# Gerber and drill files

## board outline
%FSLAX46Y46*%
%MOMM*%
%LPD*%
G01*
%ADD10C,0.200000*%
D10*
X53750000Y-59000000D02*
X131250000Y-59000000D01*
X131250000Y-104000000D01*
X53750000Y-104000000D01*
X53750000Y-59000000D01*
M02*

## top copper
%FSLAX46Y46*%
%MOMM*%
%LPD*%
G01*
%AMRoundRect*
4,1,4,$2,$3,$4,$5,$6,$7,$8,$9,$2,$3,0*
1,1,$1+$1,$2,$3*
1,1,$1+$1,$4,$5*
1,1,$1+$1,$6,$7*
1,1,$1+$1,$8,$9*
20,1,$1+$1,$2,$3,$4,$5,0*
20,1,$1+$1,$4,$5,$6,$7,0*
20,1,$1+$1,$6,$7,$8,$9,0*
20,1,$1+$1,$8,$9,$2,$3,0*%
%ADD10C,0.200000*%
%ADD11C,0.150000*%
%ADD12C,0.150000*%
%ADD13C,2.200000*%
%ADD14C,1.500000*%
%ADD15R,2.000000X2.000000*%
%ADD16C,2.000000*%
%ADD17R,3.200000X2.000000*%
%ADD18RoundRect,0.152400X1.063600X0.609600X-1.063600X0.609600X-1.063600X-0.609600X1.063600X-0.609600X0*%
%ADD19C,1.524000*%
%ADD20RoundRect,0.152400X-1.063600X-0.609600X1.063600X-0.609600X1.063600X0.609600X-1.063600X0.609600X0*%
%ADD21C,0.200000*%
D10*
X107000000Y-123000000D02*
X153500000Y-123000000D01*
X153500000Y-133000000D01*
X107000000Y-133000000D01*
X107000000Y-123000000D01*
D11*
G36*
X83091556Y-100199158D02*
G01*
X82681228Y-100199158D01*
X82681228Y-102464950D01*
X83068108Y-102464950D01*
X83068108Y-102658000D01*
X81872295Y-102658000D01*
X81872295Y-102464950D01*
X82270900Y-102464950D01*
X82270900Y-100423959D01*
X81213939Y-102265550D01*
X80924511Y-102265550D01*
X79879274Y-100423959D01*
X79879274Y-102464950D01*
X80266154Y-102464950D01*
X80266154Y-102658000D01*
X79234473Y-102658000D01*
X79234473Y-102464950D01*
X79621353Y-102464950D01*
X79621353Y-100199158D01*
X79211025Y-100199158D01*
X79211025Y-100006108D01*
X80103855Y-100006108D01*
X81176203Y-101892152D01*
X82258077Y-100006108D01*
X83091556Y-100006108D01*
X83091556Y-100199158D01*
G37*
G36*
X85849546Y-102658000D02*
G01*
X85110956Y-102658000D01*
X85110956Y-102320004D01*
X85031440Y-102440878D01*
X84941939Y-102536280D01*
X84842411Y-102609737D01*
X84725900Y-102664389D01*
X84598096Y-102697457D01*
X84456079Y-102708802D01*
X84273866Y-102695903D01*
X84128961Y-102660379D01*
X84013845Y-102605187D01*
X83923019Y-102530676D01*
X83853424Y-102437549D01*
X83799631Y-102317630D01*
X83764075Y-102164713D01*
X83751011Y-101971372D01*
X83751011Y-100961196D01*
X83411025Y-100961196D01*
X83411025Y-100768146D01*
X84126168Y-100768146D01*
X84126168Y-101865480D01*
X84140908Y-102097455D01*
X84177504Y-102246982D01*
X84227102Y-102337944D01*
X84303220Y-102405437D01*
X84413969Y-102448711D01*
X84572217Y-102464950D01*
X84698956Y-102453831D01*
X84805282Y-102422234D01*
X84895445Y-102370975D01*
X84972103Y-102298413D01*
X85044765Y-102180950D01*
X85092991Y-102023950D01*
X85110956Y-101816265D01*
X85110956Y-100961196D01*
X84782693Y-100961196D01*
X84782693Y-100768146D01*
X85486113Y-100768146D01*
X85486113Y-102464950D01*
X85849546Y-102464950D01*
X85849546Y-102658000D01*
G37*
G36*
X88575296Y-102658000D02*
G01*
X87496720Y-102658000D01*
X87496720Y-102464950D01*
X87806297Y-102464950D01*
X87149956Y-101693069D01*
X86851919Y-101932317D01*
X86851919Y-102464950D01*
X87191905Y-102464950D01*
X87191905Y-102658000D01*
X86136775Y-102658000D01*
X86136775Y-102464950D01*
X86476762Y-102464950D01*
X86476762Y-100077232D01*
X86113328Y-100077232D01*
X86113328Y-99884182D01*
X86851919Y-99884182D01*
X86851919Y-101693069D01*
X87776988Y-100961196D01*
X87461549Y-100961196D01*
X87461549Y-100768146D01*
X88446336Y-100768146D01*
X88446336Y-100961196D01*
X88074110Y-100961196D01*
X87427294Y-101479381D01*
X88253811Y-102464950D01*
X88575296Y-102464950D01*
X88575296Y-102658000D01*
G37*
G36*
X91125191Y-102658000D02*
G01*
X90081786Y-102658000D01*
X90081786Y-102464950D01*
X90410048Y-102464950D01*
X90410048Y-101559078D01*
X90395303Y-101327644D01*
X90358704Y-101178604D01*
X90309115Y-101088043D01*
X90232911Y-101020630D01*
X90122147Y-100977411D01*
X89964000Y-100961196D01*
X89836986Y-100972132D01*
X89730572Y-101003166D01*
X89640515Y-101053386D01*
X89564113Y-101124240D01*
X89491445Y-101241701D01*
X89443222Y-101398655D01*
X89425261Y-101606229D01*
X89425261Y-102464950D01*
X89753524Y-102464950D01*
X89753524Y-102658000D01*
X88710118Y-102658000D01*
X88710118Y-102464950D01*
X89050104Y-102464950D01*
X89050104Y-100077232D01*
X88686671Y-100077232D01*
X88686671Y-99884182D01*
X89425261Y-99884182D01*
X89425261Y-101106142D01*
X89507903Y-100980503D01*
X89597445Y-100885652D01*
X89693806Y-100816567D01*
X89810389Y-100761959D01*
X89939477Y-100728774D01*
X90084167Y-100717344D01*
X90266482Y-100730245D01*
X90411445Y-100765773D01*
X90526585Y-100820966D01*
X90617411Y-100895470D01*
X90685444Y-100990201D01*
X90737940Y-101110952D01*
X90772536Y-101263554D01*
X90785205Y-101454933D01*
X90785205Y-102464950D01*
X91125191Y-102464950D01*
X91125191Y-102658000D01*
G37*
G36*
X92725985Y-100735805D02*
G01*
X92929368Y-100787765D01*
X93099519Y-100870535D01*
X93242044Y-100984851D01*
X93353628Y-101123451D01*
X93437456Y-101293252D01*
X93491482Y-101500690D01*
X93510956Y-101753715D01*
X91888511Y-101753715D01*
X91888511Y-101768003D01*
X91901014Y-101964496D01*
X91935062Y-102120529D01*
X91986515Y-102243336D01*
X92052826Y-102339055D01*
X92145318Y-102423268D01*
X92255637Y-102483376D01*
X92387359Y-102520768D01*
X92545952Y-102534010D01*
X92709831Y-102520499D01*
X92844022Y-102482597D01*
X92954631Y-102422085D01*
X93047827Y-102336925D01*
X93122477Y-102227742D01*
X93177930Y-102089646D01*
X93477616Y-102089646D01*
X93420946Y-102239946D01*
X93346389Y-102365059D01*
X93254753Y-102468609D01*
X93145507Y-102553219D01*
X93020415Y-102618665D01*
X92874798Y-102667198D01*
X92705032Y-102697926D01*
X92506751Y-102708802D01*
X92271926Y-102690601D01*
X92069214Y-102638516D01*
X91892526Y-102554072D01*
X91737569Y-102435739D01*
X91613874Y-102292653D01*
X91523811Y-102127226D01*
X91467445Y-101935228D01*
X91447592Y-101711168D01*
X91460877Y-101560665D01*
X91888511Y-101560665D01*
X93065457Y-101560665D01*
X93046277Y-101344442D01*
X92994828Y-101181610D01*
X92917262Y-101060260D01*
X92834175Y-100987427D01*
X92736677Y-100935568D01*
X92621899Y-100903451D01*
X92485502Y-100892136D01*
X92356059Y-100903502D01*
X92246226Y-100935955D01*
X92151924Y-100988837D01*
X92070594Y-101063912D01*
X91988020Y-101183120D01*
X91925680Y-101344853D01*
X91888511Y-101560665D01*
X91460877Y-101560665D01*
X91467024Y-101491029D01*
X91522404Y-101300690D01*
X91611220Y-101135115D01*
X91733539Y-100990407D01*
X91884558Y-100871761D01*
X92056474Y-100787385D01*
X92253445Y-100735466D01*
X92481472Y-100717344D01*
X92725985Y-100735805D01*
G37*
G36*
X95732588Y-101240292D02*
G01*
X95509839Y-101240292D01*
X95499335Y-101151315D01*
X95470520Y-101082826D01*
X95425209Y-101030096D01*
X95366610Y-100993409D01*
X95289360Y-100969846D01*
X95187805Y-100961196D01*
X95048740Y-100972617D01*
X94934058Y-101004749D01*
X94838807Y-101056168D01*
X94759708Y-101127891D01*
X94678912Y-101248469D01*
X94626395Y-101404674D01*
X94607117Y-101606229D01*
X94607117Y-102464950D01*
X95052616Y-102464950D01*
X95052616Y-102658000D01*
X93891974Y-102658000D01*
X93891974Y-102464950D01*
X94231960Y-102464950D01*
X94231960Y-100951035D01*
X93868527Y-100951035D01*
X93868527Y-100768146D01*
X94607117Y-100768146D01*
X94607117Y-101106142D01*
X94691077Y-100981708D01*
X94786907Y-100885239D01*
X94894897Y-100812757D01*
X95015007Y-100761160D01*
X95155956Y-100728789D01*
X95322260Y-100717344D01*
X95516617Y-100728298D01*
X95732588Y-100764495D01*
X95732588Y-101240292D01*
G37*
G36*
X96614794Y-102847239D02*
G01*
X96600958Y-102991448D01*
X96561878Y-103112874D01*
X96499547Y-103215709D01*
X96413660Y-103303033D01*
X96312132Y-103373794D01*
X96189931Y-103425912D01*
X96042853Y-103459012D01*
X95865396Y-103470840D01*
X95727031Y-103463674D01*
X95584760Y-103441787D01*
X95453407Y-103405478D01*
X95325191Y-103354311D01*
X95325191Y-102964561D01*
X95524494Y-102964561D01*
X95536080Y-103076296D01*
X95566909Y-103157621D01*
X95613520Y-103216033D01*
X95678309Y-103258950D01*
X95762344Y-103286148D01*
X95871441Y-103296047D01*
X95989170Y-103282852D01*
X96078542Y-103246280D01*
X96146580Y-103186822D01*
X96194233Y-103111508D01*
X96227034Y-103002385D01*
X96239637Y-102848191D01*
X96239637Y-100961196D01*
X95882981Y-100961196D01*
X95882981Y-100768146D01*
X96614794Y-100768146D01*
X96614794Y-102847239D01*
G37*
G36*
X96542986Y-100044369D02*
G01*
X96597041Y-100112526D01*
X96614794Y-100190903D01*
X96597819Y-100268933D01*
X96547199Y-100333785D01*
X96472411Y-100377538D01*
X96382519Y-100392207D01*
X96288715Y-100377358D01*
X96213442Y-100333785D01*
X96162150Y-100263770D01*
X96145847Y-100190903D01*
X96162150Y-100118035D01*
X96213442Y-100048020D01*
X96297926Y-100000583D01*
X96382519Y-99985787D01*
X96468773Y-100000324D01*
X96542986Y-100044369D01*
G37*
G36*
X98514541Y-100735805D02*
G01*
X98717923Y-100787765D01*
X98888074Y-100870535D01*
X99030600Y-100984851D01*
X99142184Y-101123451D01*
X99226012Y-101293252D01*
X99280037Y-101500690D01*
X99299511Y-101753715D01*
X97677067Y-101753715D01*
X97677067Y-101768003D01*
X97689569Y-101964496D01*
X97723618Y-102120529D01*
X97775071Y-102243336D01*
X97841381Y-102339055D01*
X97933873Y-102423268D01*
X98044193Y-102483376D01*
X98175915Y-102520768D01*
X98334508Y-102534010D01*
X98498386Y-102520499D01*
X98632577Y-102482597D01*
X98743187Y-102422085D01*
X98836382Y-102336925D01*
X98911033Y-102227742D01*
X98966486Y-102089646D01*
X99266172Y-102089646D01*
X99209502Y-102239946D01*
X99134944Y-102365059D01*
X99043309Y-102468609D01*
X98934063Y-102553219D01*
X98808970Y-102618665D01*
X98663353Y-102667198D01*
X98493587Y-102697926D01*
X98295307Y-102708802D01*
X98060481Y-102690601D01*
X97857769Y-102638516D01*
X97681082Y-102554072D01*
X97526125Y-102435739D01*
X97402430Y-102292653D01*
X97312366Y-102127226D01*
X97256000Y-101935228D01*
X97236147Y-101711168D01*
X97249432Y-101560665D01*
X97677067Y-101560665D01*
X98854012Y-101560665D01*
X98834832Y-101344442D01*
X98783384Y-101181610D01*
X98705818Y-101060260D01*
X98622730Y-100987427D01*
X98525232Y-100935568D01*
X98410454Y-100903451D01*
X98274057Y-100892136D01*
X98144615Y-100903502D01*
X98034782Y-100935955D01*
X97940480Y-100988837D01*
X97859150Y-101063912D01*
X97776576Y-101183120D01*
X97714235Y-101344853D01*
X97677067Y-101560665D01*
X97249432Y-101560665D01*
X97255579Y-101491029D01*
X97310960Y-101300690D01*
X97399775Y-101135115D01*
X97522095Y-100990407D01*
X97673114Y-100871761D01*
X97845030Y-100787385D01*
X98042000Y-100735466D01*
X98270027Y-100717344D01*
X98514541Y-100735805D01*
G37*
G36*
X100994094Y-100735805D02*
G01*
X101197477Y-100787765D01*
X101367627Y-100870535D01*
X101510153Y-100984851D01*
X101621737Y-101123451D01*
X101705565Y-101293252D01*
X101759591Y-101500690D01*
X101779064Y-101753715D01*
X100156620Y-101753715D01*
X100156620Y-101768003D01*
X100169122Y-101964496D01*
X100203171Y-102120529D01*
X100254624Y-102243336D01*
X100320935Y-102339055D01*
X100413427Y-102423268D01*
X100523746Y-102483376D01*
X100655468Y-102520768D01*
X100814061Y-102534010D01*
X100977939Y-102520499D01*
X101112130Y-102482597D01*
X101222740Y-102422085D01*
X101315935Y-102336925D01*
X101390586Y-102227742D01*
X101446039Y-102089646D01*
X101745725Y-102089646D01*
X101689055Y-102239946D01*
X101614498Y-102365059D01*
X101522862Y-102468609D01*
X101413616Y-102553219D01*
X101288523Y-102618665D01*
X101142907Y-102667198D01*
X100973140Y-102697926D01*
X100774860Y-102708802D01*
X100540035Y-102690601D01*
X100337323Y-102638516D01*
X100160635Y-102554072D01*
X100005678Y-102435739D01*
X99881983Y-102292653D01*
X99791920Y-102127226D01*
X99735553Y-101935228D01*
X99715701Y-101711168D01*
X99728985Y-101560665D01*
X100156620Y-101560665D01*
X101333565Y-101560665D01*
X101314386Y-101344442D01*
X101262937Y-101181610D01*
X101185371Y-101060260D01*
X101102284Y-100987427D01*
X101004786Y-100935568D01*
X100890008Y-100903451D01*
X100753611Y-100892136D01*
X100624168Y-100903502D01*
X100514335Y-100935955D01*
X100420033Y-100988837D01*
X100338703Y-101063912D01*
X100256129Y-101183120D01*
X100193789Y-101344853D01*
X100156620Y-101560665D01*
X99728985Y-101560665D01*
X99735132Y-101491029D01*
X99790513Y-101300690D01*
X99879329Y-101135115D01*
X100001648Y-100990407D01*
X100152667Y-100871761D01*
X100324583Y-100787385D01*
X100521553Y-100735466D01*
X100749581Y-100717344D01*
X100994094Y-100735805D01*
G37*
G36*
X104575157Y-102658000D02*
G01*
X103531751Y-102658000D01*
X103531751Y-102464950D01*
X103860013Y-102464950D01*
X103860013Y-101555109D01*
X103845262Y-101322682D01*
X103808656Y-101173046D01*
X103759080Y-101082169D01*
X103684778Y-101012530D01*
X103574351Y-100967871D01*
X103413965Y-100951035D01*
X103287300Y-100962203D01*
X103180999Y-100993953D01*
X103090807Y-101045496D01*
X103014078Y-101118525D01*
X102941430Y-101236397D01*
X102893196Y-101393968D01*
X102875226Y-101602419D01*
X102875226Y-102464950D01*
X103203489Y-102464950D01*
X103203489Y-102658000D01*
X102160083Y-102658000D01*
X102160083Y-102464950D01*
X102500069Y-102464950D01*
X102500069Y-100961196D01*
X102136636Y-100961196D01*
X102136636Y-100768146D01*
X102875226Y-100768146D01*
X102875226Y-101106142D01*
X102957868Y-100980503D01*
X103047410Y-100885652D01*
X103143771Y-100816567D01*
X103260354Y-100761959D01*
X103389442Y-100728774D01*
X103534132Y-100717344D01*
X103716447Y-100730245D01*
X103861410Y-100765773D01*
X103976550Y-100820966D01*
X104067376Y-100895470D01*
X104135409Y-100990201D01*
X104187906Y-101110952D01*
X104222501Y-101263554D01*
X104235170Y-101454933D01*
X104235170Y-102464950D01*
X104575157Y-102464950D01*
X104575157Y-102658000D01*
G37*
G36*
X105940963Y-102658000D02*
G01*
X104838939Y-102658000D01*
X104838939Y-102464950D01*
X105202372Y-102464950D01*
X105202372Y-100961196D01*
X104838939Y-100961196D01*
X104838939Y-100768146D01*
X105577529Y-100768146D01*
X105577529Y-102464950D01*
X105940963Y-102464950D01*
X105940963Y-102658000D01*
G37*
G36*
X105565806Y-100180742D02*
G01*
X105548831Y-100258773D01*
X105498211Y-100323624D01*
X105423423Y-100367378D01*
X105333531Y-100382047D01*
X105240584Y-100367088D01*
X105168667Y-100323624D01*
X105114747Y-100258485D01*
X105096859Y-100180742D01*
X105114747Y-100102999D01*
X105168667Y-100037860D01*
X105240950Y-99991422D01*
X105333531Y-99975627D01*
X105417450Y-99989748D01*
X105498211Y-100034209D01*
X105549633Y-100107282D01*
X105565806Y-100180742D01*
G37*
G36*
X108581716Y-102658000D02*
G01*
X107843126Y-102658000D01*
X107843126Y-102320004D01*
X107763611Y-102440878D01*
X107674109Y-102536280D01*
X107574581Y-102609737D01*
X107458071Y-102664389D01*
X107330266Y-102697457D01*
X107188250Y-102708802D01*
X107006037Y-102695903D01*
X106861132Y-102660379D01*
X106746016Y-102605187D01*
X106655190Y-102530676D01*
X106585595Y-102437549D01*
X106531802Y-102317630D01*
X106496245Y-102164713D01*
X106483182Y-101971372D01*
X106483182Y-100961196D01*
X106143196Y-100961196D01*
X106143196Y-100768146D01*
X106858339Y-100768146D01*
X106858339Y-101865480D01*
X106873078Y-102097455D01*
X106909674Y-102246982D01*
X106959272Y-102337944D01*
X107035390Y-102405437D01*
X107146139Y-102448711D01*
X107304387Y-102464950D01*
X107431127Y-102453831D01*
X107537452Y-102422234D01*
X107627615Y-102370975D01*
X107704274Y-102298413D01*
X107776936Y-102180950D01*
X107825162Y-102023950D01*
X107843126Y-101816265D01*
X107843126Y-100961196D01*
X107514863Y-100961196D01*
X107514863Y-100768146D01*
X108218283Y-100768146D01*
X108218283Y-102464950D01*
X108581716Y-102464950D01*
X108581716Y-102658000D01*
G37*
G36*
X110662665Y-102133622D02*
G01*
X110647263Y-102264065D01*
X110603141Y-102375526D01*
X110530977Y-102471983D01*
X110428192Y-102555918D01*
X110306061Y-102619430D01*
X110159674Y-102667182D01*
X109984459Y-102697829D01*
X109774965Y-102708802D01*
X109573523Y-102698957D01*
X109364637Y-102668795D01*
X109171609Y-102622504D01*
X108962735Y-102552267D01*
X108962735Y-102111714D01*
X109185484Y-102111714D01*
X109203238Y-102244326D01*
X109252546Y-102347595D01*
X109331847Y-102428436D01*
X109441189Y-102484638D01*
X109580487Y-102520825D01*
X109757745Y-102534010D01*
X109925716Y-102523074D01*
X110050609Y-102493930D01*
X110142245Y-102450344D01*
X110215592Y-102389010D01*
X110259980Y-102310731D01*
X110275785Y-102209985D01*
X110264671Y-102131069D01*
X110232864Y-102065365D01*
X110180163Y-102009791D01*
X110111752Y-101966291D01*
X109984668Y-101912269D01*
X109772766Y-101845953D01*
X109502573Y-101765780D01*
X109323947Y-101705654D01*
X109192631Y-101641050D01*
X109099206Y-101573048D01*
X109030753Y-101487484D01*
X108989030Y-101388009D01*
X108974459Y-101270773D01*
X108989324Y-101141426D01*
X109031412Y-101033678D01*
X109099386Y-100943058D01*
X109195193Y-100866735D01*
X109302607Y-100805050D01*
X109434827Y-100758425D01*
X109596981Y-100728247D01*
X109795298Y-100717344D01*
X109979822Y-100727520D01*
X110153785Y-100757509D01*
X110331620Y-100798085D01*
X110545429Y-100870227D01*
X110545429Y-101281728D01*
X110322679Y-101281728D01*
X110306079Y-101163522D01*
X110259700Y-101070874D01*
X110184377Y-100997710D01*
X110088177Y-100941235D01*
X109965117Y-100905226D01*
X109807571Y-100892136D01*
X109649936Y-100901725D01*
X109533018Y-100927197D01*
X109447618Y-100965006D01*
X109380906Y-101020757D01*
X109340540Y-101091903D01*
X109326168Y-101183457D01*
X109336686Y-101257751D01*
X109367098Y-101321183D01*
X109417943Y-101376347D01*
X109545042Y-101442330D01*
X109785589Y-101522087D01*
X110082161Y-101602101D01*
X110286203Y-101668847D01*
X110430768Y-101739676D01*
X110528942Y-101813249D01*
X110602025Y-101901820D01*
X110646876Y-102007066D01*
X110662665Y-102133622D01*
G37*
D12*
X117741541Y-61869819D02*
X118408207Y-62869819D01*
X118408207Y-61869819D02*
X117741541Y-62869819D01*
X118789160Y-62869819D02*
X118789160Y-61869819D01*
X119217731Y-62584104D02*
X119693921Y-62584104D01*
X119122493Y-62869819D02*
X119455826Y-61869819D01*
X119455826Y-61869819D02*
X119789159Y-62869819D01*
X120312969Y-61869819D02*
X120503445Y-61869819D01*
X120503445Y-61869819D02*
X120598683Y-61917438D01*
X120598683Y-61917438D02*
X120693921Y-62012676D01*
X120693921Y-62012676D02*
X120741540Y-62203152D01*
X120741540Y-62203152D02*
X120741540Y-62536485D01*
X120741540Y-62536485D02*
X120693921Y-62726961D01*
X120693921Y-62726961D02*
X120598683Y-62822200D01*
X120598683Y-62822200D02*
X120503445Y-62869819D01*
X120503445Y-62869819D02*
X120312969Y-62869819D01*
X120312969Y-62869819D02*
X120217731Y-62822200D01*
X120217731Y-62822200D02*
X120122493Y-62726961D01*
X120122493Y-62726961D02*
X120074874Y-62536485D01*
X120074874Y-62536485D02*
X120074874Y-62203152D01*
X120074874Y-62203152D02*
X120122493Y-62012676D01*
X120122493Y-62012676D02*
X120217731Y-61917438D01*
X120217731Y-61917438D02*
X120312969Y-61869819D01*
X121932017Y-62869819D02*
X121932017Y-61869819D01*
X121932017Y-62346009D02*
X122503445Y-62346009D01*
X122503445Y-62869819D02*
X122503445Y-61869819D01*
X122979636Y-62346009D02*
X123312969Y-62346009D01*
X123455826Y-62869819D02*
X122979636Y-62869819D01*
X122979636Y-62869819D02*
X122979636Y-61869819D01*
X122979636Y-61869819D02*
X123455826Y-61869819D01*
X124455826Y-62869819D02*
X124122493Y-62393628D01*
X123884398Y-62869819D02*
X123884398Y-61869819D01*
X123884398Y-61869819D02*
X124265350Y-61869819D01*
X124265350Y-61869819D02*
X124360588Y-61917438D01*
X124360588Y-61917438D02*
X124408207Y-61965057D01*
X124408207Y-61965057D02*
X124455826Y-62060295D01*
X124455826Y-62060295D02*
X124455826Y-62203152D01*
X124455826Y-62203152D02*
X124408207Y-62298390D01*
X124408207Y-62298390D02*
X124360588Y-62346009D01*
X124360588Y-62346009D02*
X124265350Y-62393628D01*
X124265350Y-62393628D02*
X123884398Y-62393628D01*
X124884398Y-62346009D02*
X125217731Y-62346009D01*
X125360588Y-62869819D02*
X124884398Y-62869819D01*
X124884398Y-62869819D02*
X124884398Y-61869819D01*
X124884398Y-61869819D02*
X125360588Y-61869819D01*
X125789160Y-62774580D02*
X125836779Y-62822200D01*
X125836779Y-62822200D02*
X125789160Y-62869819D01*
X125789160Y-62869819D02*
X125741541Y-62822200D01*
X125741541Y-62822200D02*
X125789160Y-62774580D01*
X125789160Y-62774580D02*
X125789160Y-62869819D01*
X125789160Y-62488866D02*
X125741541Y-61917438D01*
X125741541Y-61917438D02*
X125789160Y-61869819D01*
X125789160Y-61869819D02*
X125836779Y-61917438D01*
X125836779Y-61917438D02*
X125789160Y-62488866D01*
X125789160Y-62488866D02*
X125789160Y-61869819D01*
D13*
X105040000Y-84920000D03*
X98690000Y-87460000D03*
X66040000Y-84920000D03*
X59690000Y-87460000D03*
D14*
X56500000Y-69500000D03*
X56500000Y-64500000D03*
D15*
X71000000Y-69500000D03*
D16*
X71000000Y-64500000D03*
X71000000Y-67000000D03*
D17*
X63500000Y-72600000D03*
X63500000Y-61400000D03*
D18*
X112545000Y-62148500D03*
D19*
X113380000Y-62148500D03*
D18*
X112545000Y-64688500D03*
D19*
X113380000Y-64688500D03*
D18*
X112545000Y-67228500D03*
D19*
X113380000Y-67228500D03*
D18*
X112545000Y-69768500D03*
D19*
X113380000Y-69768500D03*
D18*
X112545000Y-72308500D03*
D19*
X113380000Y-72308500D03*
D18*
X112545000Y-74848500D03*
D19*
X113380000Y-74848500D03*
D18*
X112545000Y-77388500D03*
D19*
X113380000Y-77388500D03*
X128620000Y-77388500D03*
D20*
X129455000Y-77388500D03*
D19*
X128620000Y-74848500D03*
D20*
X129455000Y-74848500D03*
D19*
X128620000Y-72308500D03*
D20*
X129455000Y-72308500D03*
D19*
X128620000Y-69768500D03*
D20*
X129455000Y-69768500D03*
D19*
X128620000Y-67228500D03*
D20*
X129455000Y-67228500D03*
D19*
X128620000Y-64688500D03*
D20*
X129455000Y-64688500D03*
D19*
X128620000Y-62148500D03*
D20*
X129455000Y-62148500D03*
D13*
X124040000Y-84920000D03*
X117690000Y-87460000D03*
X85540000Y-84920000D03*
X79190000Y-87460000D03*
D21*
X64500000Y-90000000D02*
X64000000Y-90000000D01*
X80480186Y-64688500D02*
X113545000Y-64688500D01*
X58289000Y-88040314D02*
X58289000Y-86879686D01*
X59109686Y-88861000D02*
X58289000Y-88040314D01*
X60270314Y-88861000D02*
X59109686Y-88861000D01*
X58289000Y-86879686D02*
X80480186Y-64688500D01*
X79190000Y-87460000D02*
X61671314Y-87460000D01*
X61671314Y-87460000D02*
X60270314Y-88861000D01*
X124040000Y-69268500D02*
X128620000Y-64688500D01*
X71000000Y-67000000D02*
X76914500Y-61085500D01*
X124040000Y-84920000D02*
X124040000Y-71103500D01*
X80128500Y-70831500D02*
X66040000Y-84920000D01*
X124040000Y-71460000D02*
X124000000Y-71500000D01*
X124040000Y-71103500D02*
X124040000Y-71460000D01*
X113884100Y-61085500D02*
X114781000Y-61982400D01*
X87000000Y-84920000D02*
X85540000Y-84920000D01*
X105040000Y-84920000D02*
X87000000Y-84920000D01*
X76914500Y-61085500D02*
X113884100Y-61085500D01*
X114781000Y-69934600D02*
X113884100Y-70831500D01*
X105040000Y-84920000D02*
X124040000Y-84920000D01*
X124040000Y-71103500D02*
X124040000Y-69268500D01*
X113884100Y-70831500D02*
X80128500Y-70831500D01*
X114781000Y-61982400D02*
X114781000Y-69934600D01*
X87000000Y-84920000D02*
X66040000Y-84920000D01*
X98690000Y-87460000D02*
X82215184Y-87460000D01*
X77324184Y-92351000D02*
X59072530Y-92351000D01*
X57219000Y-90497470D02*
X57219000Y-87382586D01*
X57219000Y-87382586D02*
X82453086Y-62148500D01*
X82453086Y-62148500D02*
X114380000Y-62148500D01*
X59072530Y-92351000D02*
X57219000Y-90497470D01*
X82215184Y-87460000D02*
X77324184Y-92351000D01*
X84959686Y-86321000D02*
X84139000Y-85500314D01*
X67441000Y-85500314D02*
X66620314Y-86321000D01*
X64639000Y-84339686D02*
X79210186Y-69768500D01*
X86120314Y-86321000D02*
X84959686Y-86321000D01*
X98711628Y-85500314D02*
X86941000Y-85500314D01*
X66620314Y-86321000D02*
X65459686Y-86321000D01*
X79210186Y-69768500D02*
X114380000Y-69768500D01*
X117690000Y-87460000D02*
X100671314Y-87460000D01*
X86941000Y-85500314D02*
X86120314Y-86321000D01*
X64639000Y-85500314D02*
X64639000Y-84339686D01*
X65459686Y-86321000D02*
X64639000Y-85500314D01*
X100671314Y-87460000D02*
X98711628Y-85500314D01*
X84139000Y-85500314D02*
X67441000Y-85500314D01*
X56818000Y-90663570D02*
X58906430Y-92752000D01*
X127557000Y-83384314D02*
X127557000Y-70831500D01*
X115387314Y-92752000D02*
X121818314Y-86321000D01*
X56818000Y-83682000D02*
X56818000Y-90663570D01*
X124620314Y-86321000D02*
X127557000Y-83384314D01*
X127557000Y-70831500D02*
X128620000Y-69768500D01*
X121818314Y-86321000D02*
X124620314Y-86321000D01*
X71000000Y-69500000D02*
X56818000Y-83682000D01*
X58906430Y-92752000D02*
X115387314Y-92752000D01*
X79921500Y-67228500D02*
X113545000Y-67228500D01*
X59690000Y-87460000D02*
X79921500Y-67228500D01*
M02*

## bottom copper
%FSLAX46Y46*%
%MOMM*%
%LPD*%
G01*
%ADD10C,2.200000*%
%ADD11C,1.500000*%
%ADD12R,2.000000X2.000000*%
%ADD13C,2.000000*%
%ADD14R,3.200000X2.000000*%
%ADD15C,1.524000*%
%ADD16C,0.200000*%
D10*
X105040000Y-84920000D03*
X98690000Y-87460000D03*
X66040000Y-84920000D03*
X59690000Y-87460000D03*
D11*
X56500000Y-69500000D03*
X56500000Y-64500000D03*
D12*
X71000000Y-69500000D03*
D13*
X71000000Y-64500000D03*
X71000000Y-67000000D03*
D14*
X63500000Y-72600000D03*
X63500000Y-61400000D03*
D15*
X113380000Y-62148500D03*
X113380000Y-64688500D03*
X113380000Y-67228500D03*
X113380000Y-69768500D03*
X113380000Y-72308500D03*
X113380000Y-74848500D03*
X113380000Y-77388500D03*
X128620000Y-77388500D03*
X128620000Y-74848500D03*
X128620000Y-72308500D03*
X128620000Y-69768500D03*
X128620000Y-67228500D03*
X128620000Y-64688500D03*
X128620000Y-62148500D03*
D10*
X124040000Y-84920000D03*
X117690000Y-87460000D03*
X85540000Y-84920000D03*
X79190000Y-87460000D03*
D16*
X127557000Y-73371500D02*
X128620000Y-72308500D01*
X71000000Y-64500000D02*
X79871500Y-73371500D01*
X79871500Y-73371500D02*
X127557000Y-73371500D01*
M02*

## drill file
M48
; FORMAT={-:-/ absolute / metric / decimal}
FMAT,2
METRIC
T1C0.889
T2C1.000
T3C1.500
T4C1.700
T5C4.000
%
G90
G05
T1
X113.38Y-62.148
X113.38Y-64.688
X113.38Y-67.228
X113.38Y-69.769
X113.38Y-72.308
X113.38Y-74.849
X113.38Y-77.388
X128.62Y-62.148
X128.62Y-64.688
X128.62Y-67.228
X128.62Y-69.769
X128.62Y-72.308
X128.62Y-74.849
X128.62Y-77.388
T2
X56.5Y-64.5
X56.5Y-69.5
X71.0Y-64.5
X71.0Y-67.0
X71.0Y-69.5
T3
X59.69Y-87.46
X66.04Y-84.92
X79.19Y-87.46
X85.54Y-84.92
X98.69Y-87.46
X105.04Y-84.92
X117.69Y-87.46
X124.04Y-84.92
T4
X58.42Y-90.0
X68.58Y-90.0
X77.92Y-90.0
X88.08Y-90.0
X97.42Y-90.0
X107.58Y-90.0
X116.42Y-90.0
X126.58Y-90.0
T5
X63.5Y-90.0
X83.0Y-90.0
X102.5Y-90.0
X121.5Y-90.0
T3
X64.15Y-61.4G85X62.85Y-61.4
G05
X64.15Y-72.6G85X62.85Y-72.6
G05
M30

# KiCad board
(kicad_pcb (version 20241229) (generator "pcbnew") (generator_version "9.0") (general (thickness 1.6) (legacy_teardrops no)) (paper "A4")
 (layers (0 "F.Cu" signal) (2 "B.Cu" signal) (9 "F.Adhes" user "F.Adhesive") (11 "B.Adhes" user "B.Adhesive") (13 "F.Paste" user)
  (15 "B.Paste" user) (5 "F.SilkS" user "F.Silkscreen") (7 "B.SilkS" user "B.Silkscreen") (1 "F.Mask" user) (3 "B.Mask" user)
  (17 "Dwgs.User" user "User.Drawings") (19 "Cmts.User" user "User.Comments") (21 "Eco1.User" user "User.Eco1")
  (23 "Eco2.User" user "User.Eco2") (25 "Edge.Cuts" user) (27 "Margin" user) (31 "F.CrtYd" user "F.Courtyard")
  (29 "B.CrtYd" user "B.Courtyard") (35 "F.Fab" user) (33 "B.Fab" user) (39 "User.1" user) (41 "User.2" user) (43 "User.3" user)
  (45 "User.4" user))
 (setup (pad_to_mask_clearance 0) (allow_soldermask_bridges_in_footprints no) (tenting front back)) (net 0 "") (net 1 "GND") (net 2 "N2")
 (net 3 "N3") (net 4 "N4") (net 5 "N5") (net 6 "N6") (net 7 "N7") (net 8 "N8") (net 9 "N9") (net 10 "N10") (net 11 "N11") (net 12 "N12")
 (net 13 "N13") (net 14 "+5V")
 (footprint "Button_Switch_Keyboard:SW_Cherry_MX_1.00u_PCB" (layer "F.Cu") (at 105.04 84.92)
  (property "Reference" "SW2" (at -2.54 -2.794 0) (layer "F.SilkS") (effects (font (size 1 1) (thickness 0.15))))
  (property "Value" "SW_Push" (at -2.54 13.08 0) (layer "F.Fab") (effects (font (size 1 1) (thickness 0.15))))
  (pad "" np_thru_hole circle (at -7.62 5.08) (size 1.7 1.7) (drill 1.7) (layers "*.Cu" "*.Mask"))
  (pad "" np_thru_hole circle (at -2.54 5.08) (size 4 4) (drill 4) (layers "*.Cu" "*.Mask"))
  (pad "" np_thru_hole circle (at 2.54 5.08) (size 1.7 1.7) (drill 1.7) (layers "*.Cu" "*.Mask"))
  (pad "1" thru_hole circle (at 0 0) (size 2.2 2.2) (drill 1.5) (layers "*.Cu" "*.Mask") (remove_unused_layers no) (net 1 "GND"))
  (pad "2" thru_hole circle (at -6.35 2.54) (size 2.2 2.2) (drill 1.5) (layers "*.Cu" "*.Mask") (remove_unused_layers no) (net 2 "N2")))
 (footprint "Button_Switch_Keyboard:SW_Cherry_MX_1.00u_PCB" (layer "F.Cu") (at 66.04 84.92)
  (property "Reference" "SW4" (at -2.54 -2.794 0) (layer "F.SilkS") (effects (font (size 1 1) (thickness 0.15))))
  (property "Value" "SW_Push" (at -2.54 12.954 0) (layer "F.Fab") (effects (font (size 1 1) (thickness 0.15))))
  (pad "" np_thru_hole circle (at -7.62 5.08) (size 1.7 1.7) (drill 1.7) (layers "*.Cu" "*.Mask"))
  (pad "" np_thru_hole circle (at -2.54 5.08) (size 4 4) (drill 4) (layers "*.Cu" "*.Mask"))
  (pad "" np_thru_hole circle (at 2.54 5.08) (size 1.7 1.7) (drill 1.7) (layers "*.Cu" "*.Mask"))
  (pad "1" thru_hole circle (at 0 0) (size 2.2 2.2) (drill 1.5) (layers "*.Cu" "*.Mask") (remove_unused_layers no) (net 1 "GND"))
  (pad "2" thru_hole circle (at -6.35 2.54) (size 2.2 2.2) (drill 1.5) (layers "*.Cu" "*.Mask") (remove_unused_layers no) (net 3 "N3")))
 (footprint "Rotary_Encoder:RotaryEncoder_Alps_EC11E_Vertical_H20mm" (layer "F.Cu") (at 71 69.5 180)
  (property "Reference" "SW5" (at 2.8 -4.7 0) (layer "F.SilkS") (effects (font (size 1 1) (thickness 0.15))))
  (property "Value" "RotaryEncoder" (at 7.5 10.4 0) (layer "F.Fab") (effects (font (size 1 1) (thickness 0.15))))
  (pad "" thru_hole circle (at 14.5 0 180) (size 1.5 1.5) (drill 1) (layers "*.Cu" "*.Mask") (remove_unused_layers no))
  (pad "" thru_hole circle (at 14.5 5 180) (size 1.5 1.5) (drill 1) (layers "*.Cu" "*.Mask") (remove_unused_layers no))
  (pad "A" thru_hole rect (at 0 0 180) (size 2 2) (drill 1) (layers "*.Cu" "*.Mask") (remove_unused_layers no) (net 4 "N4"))
  (pad "B" thru_hole circle (at 0 5 180) (size 2 2) (drill 1) (layers "*.Cu" "*.Mask") (remove_unused_layers no) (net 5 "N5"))
  (pad "C" thru_hole circle (at 0 2.5 180) (size 2 2) (drill 1) (layers "*.Cu" "*.Mask") (remove_unused_layers no) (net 1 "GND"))
  (pad "MP" thru_hole rect (at 7.5 -3.1 180) (size 3.2 2) (drill oval 2.8 1.5) (layers "*.Cu" "*.Mask") (remove_unused_layers no))
  (pad "MP" thru_hole rect (at 7.5 8.1 180) (size 3.2 2) (drill oval 2.8 1.5) (layers "*.Cu" "*.Mask") (remove_unused_layers no)))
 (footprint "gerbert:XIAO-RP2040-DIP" (layer "F.Cu") (at 121 69.7685)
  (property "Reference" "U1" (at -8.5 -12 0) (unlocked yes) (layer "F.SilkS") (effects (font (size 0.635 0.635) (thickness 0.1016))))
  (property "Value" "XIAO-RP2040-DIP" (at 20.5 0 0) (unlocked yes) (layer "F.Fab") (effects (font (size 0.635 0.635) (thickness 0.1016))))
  (pad "1" smd roundrect (at -8.455 -7.62 180) (size 2.432 1.524) (layers "F.Cu" "F.Mask") (roundrect_rratio 0.1) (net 2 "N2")
   (thermal_bridge_angle 45))
  (pad "1" thru_hole circle (at -7.62 -7.62 180) (size 1.524 1.524) (drill 0.889) (layers "*.Cu" "*.Mask") (remove_unused_layers no)
   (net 2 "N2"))
  (pad "2" smd roundrect (at -8.455 -5.08 180) (size 2.432 1.524) (layers "F.Cu" "F.Mask") (roundrect_rratio 0.1) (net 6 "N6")
   (thermal_bridge_angle 45))
  (pad "2" thru_hole circle (at -7.62 -5.08 180) (size 1.524 1.524) (drill 0.889) (layers "*.Cu" "*.Mask") (remove_unused_layers no)
   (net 6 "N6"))
  (pad "3" smd roundrect (at -8.455 -2.54 180) (size 2.432 1.524) (layers "F.Cu" "F.Mask") (roundrect_rratio 0.1) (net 3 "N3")
   (thermal_bridge_angle 45))
  (pad "3" thru_hole circle (at -7.62 -2.54 180) (size 1.524 1.524) (drill 0.889) (layers "*.Cu" "*.Mask") (remove_unused_layers no)
   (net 3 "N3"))
  (pad "4" smd roundrect (at -8.455 0 180) (size 2.432 1.524) (layers "F.Cu" "F.Mask") (roundrect_rratio 0.1) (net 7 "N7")
   (thermal_bridge_angle 45))
  (pad "4" thru_hole circle (at -7.62 0 180) (size 1.524 1.524) (drill 0.889) (layers "*.Cu" "*.Mask") (remove_unused_layers no)
   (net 7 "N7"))
  (pad "5" smd roundrect (at -8.455 2.54 180) (size 2.432 1.524) (layers "F.Cu" "F.Mask") (roundrect_rratio 0.1) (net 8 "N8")
   (thermal_bridge_angle 45))
  (pad "5" thru_hole circle (at -7.62 2.54 180) (size 1.524 1.524) (drill 0.889) (layers "*.Cu" "*.Mask") (remove_unused_layers no)
   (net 8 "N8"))
  (pad "6" smd roundrect (at -8.455 5.08 180) (size 2.432 1.524) (layers "F.Cu" "F.Mask") (roundrect_rratio 0.1) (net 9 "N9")
   (thermal_bridge_angle 45))
  (pad "6" thru_hole circle (at -7.62 5.08 180) (size 1.524 1.524) (drill 0.889) (layers "*.Cu" "*.Mask") (remove_unused_layers no)
   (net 9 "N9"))
  (pad "7" smd roundrect (at -8.455 7.62 180) (size 2.432 1.524) (layers "F.Cu" "F.Mask") (roundrect_rratio 0.1) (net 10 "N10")
   (thermal_bridge_angle 45))
  (pad "7" thru_hole circle (at -7.62 7.62 180) (size 1.524 1.524) (drill 0.889) (layers "*.Cu" "*.Mask") (remove_unused_layers no)
   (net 10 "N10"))
  (pad "8" thru_hole circle (at 7.62 7.62) (size 1.524 1.524) (drill 0.889) (layers "*.Cu" "*.Mask") (remove_unused_layers no)
   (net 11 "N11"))
  (pad "8" smd roundrect (at 8.455 7.62) (size 2.432 1.524) (layers "F.Cu" "F.Mask") (roundrect_rratio 0.1) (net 11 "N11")
   (thermal_bridge_angle 45))
  (pad "9" thru_hole circle (at 7.62 5.08) (size 1.524 1.524) (drill 0.889) (layers "*.Cu" "*.Mask") (remove_unused_layers no)
   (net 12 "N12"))
  (pad "9" smd roundrect (at 8.455 5.08) (size 2.432 1.524) (layers "F.Cu" "F.Mask") (roundrect_rratio 0.1) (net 12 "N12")
   (thermal_bridge_angle 45))
  (pad "10" thru_hole circle (at 7.62 2.54) (size 1.524 1.524) (drill 0.889) (layers "*.Cu" "*.Mask") (remove_unused_layers no) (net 5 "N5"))
  (pad "10" smd roundrect (at 8.455 2.54) (size 2.432 1.524) (layers "F.Cu" "F.Mask") (roundrect_rratio 0.1) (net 5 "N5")
   (thermal_bridge_angle 45))
  (pad "11" thru_hole circle (at 7.62 0) (size 1.524 1.524) (drill 0.889) (layers "*.Cu" "*.Mask") (remove_unused_layers no) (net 4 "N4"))
  (pad "11" smd roundrect (at 8.455 0) (size 2.432 1.524) (layers "F.Cu" "F.Mask") (roundrect_rratio 0.1) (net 4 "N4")
   (thermal_bridge_angle 45))
  (pad "12" thru_hole circle (at 7.62 -2.54) (size 1.524 1.524) (drill 0.889) (layers "*.Cu" "*.Mask") (remove_unused_layers no)
   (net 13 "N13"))
  (pad "12" smd roundrect (at 8.455 -2.54) (size 2.432 1.524) (layers "F.Cu" "F.Mask") (roundrect_rratio 0.1) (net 13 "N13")
   (thermal_bridge_angle 45))
  (pad "13" thru_hole circle (at 7.62 -5.08) (size 1.524 1.524) (drill 0.889) (layers "*.Cu" "*.Mask") (remove_unused_layers no)
   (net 1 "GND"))
  (pad "13" smd roundrect (at 8.455 -5.08) (size 2.432 1.524) (layers "F.Cu" "F.Mask") (roundrect_rratio 0.1) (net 1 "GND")
   (thermal_bridge_angle 45))
  (pad "14" thru_hole circle (at 7.62 -7.62) (size 1.524 1.524) (drill 0.889) (layers "*.Cu" "*.Mask") (remove_unused_layers no)
   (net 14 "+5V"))
  (pad "14" smd roundrect (at 8.455 -7.62) (size 2.432 1.524) (layers "F.Cu" "F.Mask") (roundrect_rratio 0.1) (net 14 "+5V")
   (thermal_bridge_angle 45)))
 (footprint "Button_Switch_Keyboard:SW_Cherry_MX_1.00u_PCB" (layer "F.Cu") (at 124.04 84.92)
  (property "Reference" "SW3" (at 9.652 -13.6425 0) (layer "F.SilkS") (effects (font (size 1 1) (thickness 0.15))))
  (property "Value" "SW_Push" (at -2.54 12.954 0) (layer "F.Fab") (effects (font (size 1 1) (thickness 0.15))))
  (pad "" np_thru_hole circle (at -7.62 5.08) (size 1.7 1.7) (drill 1.7) (layers "*.Cu" "*.Mask"))
  (pad "" np_thru_hole circle (at -2.54 5.08) (size 4 4) (drill 4) (layers "*.Cu" "*.Mask"))
  (pad "" np_thru_hole circle (at 2.54 5.08) (size 1.7 1.7) (drill 1.7) (layers "*.Cu" "*.Mask"))
  (pad "1" thru_hole circle (at 0 0) (size 2.2 2.2) (drill 1.5) (layers "*.Cu" "*.Mask") (remove_unused_layers no) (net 1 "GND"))
  (pad "2" thru_hole circle (at -6.35 2.54) (size 2.2 2.2) (drill 1.5) (layers "*.Cu" "*.Mask") (remove_unused_layers no) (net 7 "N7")))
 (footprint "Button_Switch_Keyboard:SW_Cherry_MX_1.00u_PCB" (layer "F.Cu") (at 85.54 84.92)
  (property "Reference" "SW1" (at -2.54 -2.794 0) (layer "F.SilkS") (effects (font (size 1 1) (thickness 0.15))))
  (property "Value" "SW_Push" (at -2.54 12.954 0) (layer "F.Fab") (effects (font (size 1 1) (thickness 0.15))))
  (pad "" np_thru_hole circle (at -7.62 5.08) (size 1.7 1.7) (drill 1.7) (layers "*.Cu" "*.Mask"))
  (pad "" np_thru_hole circle (at -2.54 5.08) (size 4 4) (drill 4) (layers "*.Cu" "*.Mask"))
  (pad "" np_thru_hole circle (at 2.54 5.08) (size 1.7 1.7) (drill 1.7) (layers "*.Cu" "*.Mask"))
  (pad "1" thru_hole circle (at 0 0) (size 2.2 2.2) (drill 1.5) (layers "*.Cu" "*.Mask") (remove_unused_layers no) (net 1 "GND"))
  (pad "2" thru_hole circle (at -6.35 2.54) (size 2.2 2.2) (drill 1.5) (layers "*.Cu" "*.Mask") (remove_unused_layers no) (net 6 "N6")))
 (gr_rect (start 107 123) (end 153.5 133) (stroke (width 0.2) (type default)) (fill no) (layer "F.Cu"))
 (gr_rect (start 53.75 59) (end 131.25 104) (stroke (width 0.2) (type solid)) (fill no) (layer "Edge.Cuts"))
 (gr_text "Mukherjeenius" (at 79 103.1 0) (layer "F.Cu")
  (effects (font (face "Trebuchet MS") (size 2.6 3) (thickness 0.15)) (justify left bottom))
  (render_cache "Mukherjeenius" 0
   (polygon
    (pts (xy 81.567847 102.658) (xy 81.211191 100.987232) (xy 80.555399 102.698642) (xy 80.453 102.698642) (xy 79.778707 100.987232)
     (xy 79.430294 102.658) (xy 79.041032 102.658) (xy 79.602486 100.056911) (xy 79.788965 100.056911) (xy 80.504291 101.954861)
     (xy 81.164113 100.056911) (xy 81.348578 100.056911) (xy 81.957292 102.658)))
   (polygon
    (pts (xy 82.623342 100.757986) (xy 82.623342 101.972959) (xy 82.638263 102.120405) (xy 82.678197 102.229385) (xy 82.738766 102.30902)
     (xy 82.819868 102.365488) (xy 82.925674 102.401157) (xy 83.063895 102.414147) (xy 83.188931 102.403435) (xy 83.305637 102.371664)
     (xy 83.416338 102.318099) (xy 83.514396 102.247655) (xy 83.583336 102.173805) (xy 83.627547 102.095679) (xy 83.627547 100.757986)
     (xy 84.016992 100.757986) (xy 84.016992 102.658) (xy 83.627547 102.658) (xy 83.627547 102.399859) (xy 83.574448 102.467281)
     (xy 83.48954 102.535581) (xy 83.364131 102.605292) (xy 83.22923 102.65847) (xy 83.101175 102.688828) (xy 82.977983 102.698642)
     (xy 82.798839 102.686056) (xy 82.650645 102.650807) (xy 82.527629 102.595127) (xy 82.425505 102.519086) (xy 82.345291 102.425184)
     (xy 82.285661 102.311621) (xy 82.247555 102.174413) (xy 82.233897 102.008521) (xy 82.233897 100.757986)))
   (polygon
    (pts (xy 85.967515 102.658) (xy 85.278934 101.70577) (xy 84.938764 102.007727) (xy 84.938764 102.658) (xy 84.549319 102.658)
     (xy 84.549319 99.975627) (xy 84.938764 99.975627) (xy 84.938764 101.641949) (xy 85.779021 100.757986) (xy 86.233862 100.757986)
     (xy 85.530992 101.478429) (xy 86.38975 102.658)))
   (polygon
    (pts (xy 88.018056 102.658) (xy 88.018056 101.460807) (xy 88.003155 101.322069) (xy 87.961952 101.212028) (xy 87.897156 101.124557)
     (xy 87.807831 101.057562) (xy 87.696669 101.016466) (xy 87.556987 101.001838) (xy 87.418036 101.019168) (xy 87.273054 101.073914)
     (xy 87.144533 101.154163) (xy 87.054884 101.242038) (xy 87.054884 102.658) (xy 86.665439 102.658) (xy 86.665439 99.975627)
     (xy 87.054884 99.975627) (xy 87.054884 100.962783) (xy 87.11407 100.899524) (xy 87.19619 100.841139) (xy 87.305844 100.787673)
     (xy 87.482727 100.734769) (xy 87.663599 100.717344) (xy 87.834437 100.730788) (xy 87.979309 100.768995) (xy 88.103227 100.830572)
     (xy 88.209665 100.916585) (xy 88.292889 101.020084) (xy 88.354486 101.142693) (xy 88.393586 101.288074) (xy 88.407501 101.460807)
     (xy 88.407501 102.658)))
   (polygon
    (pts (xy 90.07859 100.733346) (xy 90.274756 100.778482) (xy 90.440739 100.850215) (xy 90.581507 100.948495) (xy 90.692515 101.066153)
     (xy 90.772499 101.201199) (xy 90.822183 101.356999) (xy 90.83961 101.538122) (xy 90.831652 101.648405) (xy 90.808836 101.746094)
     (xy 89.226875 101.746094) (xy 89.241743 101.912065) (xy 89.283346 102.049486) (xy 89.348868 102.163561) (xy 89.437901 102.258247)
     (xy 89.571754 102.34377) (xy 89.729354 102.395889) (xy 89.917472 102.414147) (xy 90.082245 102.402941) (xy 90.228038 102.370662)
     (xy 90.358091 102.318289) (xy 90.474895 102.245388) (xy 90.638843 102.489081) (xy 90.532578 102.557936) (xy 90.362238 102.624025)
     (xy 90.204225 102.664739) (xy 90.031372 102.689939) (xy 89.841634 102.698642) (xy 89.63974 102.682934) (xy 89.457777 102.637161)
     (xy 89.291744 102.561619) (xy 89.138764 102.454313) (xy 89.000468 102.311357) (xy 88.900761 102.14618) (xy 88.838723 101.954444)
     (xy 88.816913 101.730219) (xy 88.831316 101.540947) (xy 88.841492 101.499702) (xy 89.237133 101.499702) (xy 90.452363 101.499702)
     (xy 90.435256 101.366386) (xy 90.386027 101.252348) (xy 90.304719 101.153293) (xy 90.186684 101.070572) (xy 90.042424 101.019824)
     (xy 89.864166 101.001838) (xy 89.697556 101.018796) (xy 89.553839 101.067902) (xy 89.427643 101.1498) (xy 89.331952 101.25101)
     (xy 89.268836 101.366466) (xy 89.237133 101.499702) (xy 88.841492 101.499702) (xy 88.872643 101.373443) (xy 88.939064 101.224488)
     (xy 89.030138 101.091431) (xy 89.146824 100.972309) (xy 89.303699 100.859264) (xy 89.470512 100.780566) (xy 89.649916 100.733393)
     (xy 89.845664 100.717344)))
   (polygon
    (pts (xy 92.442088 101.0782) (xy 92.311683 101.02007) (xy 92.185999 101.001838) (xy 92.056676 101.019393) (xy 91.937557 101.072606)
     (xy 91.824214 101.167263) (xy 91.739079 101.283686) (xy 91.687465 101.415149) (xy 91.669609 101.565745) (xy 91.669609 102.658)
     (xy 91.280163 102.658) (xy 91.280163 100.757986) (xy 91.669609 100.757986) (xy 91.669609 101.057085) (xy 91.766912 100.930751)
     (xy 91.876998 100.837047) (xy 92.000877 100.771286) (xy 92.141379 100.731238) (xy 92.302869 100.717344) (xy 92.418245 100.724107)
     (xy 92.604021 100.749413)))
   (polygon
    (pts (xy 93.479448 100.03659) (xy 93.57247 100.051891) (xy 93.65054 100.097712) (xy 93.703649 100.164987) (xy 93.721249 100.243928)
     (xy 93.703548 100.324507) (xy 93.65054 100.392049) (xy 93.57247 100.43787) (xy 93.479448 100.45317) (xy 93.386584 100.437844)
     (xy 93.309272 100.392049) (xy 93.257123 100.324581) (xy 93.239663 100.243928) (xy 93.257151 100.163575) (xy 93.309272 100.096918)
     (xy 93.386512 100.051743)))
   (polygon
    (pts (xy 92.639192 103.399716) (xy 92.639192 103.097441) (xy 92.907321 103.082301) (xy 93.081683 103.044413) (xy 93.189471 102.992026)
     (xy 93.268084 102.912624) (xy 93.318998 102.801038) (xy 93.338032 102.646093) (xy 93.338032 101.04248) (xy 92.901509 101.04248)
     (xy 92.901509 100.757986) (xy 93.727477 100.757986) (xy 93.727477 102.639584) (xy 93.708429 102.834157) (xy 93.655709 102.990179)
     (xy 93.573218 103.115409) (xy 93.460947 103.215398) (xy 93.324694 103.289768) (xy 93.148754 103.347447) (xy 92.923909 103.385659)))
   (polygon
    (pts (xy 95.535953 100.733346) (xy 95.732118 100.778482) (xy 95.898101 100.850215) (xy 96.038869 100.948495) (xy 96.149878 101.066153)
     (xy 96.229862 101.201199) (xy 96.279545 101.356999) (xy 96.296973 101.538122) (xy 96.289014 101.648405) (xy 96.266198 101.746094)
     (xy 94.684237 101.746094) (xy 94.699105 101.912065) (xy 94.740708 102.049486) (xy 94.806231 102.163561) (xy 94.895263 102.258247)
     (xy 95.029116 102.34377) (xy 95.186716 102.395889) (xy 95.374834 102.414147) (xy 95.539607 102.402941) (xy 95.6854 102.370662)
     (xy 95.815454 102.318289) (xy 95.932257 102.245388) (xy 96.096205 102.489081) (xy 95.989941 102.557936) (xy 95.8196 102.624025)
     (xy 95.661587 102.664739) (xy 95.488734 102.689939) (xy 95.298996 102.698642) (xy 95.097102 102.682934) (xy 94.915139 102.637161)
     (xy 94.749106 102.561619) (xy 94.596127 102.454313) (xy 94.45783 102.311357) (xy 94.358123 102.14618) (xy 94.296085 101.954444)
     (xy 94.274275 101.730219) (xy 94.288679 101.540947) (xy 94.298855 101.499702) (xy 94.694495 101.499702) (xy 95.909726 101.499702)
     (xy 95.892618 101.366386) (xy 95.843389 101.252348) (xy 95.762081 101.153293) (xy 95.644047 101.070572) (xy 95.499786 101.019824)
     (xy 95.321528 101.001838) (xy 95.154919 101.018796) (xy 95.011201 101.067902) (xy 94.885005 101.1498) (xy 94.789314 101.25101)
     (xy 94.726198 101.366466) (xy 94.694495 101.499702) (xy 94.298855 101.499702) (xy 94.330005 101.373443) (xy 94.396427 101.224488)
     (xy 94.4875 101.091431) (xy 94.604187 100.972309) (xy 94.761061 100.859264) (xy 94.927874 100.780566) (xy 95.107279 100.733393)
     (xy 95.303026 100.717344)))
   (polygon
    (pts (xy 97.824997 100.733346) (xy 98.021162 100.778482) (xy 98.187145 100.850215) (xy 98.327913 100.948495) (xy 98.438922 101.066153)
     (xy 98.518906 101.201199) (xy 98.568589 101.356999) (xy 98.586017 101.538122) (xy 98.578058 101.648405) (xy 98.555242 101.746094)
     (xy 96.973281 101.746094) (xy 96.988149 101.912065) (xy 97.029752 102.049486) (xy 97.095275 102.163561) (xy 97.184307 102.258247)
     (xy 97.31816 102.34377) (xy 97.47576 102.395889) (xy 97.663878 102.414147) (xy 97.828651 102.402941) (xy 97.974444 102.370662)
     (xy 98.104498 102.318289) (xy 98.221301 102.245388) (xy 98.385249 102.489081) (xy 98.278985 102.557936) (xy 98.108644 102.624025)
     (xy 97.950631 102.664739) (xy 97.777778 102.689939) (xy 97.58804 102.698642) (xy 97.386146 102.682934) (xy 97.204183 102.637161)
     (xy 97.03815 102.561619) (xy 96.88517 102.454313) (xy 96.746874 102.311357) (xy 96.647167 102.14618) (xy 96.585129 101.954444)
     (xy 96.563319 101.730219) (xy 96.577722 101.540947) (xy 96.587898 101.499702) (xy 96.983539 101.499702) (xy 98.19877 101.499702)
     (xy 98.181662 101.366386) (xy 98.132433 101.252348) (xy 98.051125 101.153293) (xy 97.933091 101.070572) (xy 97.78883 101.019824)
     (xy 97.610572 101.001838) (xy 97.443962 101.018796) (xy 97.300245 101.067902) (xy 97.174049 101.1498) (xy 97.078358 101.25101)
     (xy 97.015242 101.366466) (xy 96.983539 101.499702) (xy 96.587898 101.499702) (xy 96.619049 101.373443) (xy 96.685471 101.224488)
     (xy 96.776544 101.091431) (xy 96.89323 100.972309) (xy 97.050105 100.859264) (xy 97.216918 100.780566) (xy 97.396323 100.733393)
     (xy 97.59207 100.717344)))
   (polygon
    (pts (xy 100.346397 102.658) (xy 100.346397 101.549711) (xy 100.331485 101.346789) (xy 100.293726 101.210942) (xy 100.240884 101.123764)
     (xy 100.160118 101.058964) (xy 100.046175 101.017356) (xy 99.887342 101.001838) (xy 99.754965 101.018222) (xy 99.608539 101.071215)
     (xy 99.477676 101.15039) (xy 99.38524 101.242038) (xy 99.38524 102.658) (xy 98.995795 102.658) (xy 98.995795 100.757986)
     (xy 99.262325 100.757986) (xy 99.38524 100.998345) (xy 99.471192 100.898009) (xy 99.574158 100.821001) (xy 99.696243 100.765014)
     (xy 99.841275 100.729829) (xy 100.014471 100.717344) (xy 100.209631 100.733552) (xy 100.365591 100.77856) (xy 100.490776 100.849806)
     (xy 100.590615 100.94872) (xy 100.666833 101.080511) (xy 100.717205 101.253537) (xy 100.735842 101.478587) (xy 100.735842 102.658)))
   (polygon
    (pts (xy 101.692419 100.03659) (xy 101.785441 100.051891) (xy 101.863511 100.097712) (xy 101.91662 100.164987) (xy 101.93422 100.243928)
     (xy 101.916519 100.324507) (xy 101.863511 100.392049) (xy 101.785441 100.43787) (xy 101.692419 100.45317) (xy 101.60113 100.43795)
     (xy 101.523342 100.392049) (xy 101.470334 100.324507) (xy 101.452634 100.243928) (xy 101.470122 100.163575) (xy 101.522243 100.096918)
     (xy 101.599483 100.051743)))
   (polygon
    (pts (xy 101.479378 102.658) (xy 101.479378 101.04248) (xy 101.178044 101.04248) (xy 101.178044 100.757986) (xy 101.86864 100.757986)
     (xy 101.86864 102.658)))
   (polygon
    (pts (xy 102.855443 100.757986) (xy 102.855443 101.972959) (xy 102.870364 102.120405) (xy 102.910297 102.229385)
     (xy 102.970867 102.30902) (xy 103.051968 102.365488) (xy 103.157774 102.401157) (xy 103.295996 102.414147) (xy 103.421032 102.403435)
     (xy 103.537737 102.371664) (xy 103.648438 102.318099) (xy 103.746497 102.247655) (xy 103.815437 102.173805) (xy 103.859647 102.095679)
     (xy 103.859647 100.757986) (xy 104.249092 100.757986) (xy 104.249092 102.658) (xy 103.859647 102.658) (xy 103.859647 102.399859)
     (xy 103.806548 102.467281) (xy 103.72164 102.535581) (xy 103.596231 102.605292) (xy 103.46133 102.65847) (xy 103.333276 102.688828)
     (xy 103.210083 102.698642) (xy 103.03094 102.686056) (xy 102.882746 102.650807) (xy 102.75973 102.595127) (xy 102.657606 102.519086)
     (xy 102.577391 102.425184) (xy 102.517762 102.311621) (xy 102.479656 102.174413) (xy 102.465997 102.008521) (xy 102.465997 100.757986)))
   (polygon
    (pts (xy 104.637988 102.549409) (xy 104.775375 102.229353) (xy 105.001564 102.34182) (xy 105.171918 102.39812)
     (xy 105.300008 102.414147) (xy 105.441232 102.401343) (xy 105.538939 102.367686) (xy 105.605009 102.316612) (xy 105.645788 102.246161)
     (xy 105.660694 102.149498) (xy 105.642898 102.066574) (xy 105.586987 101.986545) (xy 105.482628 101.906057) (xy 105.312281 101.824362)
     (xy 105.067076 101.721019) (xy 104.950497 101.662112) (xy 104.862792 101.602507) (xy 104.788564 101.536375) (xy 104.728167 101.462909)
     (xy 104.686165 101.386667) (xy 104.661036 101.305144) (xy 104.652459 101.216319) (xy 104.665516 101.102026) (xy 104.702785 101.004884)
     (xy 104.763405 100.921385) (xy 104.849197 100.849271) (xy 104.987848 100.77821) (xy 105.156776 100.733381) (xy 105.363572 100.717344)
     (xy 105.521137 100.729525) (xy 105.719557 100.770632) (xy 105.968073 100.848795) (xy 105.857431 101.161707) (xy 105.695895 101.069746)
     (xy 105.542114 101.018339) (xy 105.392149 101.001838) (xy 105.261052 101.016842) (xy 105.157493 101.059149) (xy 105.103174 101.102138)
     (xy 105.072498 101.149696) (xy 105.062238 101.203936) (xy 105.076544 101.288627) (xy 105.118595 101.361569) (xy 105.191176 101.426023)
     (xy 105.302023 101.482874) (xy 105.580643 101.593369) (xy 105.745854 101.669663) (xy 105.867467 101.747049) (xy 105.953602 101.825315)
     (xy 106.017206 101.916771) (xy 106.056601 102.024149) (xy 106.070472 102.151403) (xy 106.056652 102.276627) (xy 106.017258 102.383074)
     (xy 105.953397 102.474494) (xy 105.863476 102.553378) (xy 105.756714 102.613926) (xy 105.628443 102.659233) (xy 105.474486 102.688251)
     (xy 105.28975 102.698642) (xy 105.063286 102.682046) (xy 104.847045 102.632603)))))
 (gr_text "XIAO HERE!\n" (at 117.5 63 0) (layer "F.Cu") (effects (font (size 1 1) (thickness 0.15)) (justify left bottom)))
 (segment (start 64.5 90) (end 64 90) (width 0.2) (layer "F.Cu") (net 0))
 (segment (start 80.480186 64.6885) (end 113.545 64.6885) (width 0.2) (layer "F.Cu") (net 6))
 (segment (start 58.289 88.040314) (end 58.289 86.879686) (width 0.2) (layer "F.Cu") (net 6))
 (segment (start 59.109686 88.861) (end 58.289 88.040314) (width 0.2) (layer "F.Cu") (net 6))
 (segment (start 60.270314 88.861) (end 59.109686 88.861) (width 0.2) (layer "F.Cu") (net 6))
 (segment (start 58.289 86.879686) (end 80.480186 64.6885) (width 0.2) (layer "F.Cu") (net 6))
 (segment (start 79.19 87.46) (end 61.671314 87.46) (width 0.2) (layer "F.Cu") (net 6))
 (segment (start 61.671314 87.46) (end 60.270314 88.861) (width 0.2) (layer "F.Cu") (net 6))
 (segment (start 124.04 69.2685) (end 128.62 64.6885) (width 0.2) (layer "F.Cu") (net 1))
 (segment (start 71 67) (end 76.9145 61.0855) (width 0.2) (layer "F.Cu") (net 1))
 (segment (start 124.04 84.92) (end 124.04 71.1035) (width 0.2) (layer "F.Cu") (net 1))
 (segment (start 80.1285 70.8315) (end 66.04 84.92) (width 0.2) (layer "F.Cu") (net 1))
 (segment (start 124.04 71.46) (end 124 71.5) (width 0.2) (layer "F.Cu") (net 1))
 (segment (start 124.04 71.1035) (end 124.04 71.46) (width 0.2) (layer "F.Cu") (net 1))
 (segment (start 113.8841 61.0855) (end 114.781 61.9824) (width 0.2) (layer "F.Cu") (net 1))
 (segment (start 87 84.92) (end 85.54 84.92) (width 0.2) (layer "F.Cu") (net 1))
 (segment (start 105.04 84.92) (end 87 84.92) (width 0.2) (layer "F.Cu") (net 1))
 (segment (start 76.9145 61.0855) (end 113.8841 61.0855) (width 0.2) (layer "F.Cu") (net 1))
 (segment (start 114.781 69.9346) (end 113.8841 70.8315) (width 0.2) (layer "F.Cu") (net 1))
 (segment (start 105.04 84.92) (end 124.04 84.92) (width 0.2) (layer "F.Cu") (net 1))
 (segment (start 124.04 71.1035) (end 124.04 69.2685) (width 0.2) (layer "F.Cu") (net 1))
 (segment (start 113.8841 70.8315) (end 80.1285 70.8315) (width 0.2) (layer "F.Cu") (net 1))
 (segment (start 114.781 61.9824) (end 114.781 69.9346) (width 0.2) (layer "F.Cu") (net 1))
 (segment (start 87 84.92) (end 66.04 84.92) (width 0.2) (layer "F.Cu") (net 1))
 (segment (start 98.69 87.46) (end 82.215184 87.46) (width 0.2) (layer "F.Cu") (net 2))
 (segment (start 77.324184 92.351) (end 59.07253 92.351) (width 0.2) (layer "F.Cu") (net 2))
 (segment (start 57.219 90.49747) (end 57.219 87.382586) (width 0.2) (layer "F.Cu") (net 2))
 (segment (start 57.219 87.382586) (end 82.453086 62.1485) (width 0.2) (layer "F.Cu") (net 2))
 (segment (start 82.453086 62.1485) (end 114.38 62.1485) (width 0.2) (layer "F.Cu") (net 2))
 (segment (start 59.07253 92.351) (end 57.219 90.49747) (width 0.2) (layer "F.Cu") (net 2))
 (segment (start 82.215184 87.46) (end 77.324184 92.351) (width 0.2) (layer "F.Cu") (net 2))
 (segment (start 84.959686 86.321) (end 84.139 85.500314) (width 0.2) (layer "F.Cu") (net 7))
 (segment (start 67.441 85.500314) (end 66.620314 86.321) (width 0.2) (layer "F.Cu") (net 7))
 (segment (start 64.639 84.339686) (end 79.210186 69.7685) (width 0.2) (layer "F.Cu") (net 7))
 (segment (start 86.120314 86.321) (end 84.959686 86.321) (width 0.2) (layer "F.Cu") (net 7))
 (segment (start 98.711628 85.500314) (end 86.941 85.500314) (width 0.2) (layer "F.Cu") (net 7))
 (segment (start 66.620314 86.321) (end 65.459686 86.321) (width 0.2) (layer "F.Cu") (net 7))
 (segment (start 79.210186 69.7685) (end 114.38 69.7685) (width 0.2) (layer "F.Cu") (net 7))
 (segment (start 117.69 87.46) (end 100.671314 87.46) (width 0.2) (layer "F.Cu") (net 7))
 (segment (start 86.941 85.500314) (end 86.120314 86.321) (width 0.2) (layer "F.Cu") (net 7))
 (segment (start 64.639 85.500314) (end 64.639 84.339686) (width 0.2) (layer "F.Cu") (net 7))
 (segment (start 65.459686 86.321) (end 64.639 85.500314) (width 0.2) (layer "F.Cu") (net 7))
 (segment (start 100.671314 87.46) (end 98.711628 85.500314) (width 0.2) (layer "F.Cu") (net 7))
 (segment (start 84.139 85.500314) (end 67.441 85.500314) (width 0.2) (layer "F.Cu") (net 7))
 (segment (start 127.557 73.3715) (end 128.62 72.3085) (width 0.2) (layer "B.Cu") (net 5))
 (segment (start 71 64.5) (end 79.8715 73.3715) (width 0.2) (layer "B.Cu") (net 5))
 (segment (start 79.8715 73.3715) (end 127.557 73.3715) (width 0.2) (layer "B.Cu") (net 5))
 (segment (start 56.818 90.66357) (end 58.90643 92.752) (width 0.2) (layer "F.Cu") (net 4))
 (segment (start 127.557 83.384314) (end 127.557 70.8315) (width 0.2) (layer "F.Cu") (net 4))
 (segment (start 115.387314 92.752) (end 121.818314 86.321) (width 0.2) (layer "F.Cu") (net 4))
 (segment (start 56.818 83.682) (end 56.818 90.66357) (width 0.2) (layer "F.Cu") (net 4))
 (segment (start 124.620314 86.321) (end 127.557 83.384314) (width 0.2) (layer "F.Cu") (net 4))
 (segment (start 127.557 70.8315) (end 128.62 69.7685) (width 0.2) (layer "F.Cu") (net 4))
 (segment (start 121.818314 86.321) (end 124.620314 86.321) (width 0.2) (layer "F.Cu") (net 4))
 (segment (start 71 69.5) (end 56.818 83.682) (width 0.2) (layer "F.Cu") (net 4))
 (segment (start 58.90643 92.752) (end 115.387314 92.752) (width 0.2) (layer "F.Cu") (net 4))
 (segment (start 79.9215 67.2285) (end 113.545 67.2285) (width 0.2) (layer "F.Cu") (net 3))
 (segment (start 59.69 87.46) (end 79.9215 67.2285) (width 0.2) (layer "F.Cu") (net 3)))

